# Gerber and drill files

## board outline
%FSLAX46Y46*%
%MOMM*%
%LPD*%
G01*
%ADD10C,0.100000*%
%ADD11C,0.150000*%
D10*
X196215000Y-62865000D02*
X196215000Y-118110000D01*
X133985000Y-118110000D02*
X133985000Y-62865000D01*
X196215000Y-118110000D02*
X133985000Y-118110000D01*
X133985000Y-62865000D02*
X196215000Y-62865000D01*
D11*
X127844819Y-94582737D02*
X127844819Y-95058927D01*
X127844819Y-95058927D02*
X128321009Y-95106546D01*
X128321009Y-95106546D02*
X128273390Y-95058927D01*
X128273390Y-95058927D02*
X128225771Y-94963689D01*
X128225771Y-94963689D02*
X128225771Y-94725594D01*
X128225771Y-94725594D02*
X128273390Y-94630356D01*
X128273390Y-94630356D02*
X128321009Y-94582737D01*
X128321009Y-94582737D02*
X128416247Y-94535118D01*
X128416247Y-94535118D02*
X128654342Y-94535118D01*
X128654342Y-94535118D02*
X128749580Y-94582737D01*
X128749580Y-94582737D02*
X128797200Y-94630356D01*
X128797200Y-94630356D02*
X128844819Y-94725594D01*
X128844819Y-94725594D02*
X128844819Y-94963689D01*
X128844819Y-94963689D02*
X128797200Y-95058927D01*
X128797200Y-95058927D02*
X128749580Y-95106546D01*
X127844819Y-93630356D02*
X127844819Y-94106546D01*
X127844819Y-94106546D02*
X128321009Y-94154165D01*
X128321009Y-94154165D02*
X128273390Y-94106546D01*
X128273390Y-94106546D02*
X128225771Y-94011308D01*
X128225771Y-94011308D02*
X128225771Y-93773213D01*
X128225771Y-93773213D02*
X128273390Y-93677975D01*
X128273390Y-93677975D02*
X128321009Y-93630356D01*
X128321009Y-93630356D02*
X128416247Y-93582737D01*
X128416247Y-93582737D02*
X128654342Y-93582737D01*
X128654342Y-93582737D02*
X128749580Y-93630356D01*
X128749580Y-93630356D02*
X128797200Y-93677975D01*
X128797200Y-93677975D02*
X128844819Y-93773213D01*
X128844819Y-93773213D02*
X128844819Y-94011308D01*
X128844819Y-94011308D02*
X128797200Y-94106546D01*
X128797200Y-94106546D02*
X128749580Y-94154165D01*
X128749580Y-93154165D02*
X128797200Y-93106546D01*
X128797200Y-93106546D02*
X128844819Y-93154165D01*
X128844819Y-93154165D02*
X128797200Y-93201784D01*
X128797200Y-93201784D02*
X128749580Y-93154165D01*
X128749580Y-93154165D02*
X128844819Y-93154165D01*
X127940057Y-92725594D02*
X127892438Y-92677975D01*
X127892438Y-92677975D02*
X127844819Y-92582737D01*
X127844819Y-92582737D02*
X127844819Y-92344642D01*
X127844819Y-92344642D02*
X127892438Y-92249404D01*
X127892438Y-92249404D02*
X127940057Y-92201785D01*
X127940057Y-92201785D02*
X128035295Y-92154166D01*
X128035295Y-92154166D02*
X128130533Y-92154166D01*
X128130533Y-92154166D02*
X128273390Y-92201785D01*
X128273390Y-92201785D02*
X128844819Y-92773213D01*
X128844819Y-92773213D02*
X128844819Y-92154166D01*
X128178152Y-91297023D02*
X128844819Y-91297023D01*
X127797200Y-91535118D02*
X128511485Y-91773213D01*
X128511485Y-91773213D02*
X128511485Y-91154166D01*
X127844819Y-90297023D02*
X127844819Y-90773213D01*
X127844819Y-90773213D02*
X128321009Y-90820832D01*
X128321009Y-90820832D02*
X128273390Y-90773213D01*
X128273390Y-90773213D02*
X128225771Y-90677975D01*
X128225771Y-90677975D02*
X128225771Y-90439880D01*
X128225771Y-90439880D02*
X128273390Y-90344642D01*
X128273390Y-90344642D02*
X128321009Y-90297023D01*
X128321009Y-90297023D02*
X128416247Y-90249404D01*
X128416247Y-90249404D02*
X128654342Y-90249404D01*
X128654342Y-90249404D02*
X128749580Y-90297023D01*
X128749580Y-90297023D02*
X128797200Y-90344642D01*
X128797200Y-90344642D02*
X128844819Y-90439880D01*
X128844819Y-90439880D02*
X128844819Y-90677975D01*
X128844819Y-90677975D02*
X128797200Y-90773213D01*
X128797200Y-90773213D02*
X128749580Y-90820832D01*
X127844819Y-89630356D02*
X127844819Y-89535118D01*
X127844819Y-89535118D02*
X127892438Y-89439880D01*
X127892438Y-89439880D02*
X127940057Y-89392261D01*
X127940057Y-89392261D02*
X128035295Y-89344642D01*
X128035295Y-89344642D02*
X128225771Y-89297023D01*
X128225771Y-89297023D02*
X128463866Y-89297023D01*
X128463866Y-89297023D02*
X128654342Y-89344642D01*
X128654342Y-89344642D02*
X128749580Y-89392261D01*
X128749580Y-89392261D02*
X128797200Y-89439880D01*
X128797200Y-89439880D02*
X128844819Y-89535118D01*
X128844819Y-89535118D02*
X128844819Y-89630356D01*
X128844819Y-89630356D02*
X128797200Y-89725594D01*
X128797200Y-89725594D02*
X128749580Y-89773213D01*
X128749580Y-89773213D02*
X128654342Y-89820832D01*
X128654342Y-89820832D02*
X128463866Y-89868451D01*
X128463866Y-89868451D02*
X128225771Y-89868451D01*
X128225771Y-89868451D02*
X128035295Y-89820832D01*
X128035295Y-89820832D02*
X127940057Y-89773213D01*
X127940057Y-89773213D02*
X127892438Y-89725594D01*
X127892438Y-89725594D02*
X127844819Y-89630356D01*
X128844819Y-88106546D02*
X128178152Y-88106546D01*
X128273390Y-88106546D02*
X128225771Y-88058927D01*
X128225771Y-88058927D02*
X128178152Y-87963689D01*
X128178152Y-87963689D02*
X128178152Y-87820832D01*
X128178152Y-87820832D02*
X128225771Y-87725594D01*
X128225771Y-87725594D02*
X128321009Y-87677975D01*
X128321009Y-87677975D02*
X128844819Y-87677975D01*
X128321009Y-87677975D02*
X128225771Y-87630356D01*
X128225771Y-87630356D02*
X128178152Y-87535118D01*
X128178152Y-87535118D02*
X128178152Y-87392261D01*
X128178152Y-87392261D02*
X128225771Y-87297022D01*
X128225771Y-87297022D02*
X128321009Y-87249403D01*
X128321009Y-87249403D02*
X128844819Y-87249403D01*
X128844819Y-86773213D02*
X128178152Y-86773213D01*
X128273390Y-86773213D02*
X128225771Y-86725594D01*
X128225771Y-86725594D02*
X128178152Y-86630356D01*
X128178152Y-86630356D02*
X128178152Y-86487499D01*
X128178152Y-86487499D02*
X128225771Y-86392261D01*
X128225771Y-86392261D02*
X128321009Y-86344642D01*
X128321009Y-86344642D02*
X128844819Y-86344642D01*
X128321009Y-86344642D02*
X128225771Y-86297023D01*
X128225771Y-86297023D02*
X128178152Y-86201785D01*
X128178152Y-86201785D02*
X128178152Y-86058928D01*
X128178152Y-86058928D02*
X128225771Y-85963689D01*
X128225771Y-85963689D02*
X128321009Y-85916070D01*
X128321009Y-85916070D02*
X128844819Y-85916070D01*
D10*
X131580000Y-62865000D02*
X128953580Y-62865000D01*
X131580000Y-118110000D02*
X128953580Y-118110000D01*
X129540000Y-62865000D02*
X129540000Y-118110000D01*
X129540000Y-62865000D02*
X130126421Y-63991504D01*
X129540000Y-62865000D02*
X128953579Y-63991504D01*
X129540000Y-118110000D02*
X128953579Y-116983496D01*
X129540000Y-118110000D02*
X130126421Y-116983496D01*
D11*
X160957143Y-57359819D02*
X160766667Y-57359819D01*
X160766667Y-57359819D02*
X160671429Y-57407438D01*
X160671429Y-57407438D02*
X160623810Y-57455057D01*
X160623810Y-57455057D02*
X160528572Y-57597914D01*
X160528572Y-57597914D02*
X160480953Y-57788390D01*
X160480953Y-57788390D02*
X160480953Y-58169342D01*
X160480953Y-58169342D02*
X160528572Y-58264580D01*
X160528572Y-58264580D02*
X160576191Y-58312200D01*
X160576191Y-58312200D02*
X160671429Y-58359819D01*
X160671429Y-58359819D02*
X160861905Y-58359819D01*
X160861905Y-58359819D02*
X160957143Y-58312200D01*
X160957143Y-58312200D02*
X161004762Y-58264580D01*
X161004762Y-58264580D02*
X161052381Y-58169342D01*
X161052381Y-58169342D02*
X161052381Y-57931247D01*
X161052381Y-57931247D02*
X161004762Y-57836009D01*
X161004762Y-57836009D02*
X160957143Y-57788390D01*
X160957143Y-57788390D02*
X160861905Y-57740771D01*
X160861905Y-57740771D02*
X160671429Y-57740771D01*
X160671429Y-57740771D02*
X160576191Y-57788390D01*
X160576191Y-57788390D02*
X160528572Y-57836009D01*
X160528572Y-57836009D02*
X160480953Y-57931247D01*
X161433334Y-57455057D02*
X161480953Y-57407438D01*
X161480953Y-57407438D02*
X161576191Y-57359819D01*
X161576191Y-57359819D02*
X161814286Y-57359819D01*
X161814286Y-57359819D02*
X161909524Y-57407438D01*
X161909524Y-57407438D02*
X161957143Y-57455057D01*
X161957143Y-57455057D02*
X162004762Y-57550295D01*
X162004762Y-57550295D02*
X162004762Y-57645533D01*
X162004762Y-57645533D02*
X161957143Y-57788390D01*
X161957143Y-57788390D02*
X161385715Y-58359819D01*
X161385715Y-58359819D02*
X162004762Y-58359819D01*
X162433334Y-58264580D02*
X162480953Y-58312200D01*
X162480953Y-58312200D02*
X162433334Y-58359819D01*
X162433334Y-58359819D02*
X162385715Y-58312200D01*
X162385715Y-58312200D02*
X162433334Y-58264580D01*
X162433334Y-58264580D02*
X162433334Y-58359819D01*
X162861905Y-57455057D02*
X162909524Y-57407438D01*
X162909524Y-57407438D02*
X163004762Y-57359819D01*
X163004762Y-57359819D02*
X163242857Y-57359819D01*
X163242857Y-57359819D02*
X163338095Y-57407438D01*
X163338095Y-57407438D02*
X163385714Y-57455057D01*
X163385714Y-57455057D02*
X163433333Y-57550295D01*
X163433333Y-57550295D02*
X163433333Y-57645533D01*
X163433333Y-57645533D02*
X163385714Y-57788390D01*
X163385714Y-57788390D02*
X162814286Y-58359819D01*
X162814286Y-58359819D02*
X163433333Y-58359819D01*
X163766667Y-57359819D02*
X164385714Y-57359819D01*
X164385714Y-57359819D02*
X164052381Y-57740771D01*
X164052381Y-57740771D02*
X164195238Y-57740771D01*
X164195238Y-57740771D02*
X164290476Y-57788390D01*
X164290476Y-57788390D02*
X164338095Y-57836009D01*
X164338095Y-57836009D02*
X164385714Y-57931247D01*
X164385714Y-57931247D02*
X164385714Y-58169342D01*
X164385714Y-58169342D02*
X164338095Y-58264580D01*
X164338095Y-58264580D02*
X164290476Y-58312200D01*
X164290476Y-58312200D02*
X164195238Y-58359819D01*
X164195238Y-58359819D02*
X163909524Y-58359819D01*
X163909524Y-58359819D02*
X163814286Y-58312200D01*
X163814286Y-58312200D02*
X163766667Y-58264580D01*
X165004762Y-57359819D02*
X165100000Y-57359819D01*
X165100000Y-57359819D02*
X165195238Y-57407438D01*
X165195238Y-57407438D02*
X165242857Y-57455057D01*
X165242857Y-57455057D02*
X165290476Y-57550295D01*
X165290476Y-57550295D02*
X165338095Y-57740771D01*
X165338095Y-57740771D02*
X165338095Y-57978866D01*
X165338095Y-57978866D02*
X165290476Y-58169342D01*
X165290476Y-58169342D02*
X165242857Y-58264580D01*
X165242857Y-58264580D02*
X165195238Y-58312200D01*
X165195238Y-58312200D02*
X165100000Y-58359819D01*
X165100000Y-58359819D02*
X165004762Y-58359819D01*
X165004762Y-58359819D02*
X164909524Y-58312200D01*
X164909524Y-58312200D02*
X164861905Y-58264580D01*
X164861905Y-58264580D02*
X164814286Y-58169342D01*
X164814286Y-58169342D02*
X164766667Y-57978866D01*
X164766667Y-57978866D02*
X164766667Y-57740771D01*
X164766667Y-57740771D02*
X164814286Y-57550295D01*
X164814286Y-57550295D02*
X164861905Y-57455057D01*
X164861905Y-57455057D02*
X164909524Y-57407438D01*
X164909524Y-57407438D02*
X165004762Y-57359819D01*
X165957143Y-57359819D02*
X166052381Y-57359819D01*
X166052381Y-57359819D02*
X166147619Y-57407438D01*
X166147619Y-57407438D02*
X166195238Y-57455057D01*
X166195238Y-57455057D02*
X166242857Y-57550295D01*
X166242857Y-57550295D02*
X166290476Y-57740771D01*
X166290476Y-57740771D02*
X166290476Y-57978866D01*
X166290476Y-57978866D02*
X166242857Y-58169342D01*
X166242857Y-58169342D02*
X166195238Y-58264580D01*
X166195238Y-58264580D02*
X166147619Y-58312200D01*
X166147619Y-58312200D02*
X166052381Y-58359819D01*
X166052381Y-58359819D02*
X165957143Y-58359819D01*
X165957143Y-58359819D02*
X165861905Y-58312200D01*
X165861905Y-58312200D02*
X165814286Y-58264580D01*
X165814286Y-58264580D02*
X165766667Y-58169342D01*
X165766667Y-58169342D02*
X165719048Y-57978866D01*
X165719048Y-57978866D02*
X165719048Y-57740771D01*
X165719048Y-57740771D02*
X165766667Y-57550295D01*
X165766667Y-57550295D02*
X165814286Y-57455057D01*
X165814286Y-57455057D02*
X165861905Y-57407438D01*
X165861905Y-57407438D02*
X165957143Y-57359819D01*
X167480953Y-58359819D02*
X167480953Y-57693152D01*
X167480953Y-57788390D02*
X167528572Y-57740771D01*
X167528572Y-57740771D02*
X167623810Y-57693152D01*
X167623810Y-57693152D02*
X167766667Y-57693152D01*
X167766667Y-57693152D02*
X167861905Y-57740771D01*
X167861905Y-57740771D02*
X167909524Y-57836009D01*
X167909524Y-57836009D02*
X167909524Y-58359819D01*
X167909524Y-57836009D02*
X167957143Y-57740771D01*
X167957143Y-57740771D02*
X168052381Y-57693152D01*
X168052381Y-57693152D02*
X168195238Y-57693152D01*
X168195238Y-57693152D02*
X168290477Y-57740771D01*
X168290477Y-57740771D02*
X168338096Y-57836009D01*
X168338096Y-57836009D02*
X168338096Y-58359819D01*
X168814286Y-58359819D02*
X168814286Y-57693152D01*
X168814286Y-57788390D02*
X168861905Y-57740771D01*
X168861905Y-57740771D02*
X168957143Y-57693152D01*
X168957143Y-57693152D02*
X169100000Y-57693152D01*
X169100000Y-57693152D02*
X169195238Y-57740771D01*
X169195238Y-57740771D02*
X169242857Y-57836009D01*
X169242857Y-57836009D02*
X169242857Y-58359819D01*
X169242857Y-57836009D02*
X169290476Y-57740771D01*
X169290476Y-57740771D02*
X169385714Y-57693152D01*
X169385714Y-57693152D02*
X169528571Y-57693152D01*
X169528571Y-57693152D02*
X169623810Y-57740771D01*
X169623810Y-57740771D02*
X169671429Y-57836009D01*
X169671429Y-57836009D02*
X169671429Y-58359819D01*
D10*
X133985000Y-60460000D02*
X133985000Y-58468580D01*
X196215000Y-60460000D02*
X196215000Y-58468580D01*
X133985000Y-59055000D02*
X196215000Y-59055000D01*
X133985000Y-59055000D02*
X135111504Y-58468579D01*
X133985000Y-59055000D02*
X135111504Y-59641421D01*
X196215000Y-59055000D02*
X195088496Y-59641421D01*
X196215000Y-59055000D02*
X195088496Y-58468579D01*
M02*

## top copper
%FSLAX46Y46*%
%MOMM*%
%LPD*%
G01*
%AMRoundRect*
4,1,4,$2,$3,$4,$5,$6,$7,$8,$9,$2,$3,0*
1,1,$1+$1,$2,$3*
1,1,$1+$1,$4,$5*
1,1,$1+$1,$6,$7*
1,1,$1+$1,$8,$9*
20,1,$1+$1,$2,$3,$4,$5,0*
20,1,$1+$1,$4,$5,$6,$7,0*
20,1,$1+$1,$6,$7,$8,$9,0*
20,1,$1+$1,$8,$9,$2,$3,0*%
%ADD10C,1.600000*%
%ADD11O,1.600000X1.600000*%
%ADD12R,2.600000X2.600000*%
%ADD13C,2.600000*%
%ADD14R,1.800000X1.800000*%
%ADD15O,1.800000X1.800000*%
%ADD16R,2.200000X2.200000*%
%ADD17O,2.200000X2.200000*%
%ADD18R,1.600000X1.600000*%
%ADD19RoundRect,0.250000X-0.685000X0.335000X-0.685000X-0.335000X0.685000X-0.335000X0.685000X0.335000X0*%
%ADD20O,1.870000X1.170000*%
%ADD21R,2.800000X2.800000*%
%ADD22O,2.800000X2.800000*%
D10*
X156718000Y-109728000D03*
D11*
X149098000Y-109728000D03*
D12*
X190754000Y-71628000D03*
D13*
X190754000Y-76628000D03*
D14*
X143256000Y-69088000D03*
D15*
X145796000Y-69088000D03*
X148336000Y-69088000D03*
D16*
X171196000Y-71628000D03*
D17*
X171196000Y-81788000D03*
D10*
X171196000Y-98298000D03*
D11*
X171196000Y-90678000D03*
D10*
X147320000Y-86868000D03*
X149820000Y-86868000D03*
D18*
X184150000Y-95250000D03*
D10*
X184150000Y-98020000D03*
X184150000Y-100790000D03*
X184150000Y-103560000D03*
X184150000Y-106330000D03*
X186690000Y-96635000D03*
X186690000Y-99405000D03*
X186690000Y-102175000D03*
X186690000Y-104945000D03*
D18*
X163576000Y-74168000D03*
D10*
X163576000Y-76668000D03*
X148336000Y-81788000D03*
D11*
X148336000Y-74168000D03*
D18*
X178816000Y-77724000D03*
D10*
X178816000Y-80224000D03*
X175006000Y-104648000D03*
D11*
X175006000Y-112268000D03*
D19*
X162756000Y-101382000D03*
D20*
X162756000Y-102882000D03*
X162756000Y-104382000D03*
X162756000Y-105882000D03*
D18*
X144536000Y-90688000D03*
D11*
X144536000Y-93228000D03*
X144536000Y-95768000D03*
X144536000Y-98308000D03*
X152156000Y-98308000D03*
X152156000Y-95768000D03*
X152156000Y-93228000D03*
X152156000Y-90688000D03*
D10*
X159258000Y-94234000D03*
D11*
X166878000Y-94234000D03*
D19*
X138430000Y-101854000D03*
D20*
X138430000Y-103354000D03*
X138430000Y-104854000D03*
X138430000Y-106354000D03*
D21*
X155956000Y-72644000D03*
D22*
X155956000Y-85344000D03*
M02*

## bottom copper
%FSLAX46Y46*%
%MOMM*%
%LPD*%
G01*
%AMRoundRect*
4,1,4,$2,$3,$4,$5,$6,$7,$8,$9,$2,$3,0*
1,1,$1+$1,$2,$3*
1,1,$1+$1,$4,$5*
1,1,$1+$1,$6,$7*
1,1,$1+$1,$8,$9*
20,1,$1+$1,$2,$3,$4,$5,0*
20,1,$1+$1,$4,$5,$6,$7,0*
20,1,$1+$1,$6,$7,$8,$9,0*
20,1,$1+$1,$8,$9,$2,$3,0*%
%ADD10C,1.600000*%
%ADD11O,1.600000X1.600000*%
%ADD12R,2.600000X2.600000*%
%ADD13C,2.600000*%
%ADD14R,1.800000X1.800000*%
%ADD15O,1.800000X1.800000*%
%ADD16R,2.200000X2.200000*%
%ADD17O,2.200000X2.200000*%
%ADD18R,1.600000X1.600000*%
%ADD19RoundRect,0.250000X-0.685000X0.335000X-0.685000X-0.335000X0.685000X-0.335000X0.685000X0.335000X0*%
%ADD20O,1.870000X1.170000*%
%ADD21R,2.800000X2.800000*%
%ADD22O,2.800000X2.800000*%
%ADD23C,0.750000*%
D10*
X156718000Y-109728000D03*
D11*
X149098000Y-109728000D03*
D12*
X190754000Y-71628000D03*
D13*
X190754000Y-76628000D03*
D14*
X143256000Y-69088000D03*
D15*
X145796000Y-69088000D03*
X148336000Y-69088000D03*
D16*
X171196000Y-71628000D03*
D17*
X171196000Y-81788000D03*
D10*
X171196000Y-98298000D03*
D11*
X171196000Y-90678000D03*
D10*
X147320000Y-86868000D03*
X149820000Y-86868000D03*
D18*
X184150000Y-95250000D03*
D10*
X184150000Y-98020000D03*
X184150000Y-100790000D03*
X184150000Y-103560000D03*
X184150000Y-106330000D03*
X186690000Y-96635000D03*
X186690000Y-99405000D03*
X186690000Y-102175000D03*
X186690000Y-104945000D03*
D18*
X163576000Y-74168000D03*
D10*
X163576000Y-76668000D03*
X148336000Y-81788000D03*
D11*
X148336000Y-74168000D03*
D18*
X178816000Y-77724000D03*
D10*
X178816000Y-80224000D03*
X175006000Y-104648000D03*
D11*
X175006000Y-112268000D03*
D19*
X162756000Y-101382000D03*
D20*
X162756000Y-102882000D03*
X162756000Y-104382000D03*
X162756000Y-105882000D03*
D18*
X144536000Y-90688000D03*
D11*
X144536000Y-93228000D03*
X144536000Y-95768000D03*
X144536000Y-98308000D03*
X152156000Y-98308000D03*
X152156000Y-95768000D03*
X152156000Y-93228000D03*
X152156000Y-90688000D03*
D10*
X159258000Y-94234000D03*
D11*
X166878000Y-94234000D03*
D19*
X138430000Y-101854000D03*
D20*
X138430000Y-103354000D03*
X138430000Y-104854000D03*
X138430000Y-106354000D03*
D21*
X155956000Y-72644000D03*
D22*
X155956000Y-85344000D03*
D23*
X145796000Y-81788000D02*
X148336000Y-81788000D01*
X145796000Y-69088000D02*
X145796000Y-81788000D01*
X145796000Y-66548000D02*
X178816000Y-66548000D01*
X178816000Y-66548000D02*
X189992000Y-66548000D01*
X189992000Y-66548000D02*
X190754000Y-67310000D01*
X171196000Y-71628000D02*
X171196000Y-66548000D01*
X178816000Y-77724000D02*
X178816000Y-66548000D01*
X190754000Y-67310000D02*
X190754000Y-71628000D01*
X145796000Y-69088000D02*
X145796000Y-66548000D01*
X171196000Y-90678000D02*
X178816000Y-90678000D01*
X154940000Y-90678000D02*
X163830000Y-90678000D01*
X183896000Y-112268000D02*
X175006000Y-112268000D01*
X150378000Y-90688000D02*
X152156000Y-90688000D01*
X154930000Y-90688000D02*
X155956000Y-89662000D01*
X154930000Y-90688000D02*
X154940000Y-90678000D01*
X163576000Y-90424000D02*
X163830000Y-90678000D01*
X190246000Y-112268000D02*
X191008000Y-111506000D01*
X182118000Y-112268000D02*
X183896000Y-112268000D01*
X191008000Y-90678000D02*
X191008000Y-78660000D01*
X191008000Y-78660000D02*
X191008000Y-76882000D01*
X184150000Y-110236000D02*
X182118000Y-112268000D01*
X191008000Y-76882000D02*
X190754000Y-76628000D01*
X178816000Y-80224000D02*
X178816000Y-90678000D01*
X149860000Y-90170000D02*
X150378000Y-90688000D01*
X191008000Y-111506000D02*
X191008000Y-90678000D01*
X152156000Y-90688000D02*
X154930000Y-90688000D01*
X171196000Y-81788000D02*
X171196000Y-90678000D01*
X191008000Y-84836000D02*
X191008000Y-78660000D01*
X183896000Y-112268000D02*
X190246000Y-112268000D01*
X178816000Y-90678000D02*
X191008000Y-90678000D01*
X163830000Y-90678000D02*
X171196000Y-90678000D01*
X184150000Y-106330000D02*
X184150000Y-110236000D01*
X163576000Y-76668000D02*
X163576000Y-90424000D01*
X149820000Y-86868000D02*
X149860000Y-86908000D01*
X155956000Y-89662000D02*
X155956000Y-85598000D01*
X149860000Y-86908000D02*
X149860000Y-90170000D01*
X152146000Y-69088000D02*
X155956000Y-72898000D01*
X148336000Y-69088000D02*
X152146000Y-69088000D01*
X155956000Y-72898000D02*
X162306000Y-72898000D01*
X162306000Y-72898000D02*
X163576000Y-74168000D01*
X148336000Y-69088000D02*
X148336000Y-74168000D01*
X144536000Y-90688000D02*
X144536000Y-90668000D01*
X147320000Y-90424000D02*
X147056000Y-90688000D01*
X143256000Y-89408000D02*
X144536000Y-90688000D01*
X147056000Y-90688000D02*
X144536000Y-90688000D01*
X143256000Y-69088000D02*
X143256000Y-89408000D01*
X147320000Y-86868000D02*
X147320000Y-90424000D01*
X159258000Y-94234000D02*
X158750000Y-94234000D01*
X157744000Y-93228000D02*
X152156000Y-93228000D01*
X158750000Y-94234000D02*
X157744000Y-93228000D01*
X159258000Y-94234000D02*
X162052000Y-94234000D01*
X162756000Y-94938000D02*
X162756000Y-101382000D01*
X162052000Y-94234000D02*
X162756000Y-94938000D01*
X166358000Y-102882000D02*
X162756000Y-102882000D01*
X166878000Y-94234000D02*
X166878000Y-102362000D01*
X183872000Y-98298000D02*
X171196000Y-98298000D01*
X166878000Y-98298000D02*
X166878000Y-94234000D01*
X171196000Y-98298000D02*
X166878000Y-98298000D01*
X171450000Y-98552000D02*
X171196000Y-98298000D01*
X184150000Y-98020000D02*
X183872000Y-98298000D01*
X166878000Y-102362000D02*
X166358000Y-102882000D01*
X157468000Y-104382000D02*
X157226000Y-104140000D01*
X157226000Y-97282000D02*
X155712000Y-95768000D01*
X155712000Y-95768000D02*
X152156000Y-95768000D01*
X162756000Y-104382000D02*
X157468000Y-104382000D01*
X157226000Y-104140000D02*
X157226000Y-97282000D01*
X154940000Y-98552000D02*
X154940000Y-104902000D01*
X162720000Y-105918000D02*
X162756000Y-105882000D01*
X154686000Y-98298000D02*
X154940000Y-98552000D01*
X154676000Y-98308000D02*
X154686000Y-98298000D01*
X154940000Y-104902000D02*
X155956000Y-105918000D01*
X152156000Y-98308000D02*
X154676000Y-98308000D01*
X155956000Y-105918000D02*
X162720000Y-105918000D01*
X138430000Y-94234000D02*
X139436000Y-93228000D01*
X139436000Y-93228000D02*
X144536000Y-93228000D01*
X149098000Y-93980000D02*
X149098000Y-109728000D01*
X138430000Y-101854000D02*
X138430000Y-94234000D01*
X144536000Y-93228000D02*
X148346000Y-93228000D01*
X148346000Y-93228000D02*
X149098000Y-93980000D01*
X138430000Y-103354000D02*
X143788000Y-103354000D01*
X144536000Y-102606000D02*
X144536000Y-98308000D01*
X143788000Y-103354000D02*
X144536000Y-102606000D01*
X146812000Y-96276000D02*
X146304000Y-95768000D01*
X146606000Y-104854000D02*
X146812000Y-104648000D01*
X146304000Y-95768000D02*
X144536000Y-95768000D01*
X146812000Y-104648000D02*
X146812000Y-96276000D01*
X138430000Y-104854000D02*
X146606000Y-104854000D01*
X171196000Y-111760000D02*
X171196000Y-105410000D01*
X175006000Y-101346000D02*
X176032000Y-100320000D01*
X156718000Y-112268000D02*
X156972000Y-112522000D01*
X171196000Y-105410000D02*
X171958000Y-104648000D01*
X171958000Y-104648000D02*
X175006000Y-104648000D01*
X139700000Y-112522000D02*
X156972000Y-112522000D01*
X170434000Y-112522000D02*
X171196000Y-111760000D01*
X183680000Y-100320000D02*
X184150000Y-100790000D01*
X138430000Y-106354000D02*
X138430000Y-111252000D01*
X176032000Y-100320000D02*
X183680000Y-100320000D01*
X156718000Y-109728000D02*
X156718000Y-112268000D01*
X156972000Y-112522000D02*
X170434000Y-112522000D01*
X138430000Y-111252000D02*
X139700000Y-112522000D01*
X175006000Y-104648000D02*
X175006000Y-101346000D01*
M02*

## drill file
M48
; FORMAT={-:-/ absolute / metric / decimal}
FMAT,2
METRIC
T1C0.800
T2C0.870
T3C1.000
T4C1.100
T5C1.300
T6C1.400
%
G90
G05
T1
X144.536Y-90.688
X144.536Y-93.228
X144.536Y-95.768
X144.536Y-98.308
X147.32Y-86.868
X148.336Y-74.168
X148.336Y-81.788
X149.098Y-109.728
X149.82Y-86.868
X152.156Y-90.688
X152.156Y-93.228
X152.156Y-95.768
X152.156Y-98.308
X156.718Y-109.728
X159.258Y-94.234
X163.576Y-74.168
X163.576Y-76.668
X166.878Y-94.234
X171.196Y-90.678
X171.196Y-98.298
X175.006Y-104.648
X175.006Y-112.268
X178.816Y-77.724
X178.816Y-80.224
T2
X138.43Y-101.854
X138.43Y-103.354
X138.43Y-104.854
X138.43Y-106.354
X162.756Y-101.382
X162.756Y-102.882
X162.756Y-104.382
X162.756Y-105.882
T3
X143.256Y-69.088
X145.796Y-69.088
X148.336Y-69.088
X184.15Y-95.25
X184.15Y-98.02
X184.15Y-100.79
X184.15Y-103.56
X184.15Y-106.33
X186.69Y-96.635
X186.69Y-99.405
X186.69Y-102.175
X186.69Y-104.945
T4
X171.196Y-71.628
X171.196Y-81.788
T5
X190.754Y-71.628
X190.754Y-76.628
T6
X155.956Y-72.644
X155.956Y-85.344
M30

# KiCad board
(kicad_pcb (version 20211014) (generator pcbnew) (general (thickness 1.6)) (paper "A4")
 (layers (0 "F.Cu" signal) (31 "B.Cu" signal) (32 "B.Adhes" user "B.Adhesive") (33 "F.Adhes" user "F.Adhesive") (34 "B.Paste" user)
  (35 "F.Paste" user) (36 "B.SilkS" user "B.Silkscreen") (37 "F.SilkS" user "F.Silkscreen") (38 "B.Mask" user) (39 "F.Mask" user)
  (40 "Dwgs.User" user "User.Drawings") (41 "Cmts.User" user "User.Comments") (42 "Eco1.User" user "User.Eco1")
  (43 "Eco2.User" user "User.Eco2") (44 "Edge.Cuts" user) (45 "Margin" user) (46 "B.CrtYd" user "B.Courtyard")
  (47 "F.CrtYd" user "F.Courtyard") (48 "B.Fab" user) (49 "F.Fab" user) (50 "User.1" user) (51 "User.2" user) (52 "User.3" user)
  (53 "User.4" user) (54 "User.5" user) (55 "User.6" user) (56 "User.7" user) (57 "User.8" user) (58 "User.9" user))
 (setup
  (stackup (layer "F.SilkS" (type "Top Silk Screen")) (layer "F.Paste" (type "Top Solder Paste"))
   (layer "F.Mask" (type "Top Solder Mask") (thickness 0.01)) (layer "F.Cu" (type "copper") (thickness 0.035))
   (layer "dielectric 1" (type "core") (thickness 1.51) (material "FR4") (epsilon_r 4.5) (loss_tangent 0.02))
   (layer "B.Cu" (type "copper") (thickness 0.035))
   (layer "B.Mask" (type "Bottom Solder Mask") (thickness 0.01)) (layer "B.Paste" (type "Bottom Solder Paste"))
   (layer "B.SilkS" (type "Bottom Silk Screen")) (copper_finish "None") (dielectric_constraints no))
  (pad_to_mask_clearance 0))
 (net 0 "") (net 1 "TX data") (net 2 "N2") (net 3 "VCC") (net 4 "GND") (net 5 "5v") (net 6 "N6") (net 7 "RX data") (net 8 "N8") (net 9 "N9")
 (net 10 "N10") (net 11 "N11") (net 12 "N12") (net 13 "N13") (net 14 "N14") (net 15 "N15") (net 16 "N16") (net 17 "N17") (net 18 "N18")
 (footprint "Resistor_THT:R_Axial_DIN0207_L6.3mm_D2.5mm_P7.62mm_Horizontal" (layer "F.Cu") (at 156.718 109.728 180)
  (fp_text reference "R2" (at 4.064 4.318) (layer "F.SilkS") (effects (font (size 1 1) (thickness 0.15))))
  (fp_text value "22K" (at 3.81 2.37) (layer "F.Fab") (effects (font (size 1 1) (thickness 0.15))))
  (pad "1" thru_hole circle (at 0 0 180) (size 1.6 1.6) (drill 0.8) (layers *.Cu *.Mask) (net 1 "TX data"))
  (pad "2" thru_hole oval (at 7.62 0 180) (size 1.6 1.6) (drill 0.8) (layers *.Cu *.Mask) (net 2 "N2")))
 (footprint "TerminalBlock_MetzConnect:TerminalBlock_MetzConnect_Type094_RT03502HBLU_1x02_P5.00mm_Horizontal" (layer "F.Cu")
  (at 190.754 71.628 -90)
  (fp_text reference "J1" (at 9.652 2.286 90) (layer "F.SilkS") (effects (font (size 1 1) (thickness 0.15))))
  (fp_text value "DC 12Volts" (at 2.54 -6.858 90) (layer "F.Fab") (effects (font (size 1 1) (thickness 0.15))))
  (pad "1" thru_hole rect (at 0 0 270) (size 2.6 2.6) (drill 1.3) (layers *.Cu *.Mask) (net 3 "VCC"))
  (pad "2" thru_hole circle (at 5 0 270) (size 2.6 2.6) (drill 1.3) (layers *.Cu *.Mask) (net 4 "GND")))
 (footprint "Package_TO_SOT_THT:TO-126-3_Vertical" (layer "F.Cu") (at 143.256 69.088)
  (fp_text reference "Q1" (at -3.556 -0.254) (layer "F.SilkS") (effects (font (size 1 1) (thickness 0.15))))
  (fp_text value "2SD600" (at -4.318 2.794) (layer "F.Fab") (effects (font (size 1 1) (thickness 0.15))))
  (pad "1" thru_hole rect (at 0 0) (size 1.8 1.8) (drill 1) (layers *.Cu *.Mask) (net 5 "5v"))
  (pad "2" thru_hole oval (at 2.54 0) (size 1.8 1.8) (drill 1) (layers *.Cu *.Mask) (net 3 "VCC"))
  (pad "3" thru_hole oval (at 5.08 0) (size 1.8 1.8) (drill 1) (layers *.Cu *.Mask) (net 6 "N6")))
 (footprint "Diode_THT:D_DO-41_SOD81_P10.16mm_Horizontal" (layer "F.Cu") (at 171.196 71.628 -90)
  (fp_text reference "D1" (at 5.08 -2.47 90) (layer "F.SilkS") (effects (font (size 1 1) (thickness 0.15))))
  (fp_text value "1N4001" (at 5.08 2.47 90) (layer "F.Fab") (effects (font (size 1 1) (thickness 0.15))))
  (pad "1" thru_hole rect (at 0 0 270) (size 2.2 2.2) (drill 1.1) (layers *.Cu *.Mask) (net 3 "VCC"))
  (pad "2" thru_hole oval (at 10.16 0 270) (size 2.2 2.2) (drill 1.1) (layers *.Cu *.Mask) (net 4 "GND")))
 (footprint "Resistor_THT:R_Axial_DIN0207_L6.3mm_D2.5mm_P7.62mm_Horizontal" (layer "F.Cu") (at 171.196 98.298 90)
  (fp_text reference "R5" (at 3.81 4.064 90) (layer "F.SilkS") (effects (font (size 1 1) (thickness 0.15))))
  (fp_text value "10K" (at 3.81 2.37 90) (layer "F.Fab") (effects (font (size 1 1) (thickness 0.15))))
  (pad "1" thru_hole circle (at 0 0 90) (size 1.6 1.6) (drill 0.8) (layers *.Cu *.Mask) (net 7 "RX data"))
  (pad "2" thru_hole oval (at 7.62 0 90) (size 1.6 1.6) (drill 0.8) (layers *.Cu *.Mask) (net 4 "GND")))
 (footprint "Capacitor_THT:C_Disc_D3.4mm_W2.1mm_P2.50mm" (layer "F.Cu") (at 147.32 86.868)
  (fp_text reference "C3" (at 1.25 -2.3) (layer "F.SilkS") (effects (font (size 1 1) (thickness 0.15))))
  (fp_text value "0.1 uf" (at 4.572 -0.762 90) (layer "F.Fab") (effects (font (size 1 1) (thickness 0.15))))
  (pad "1" thru_hole circle (at 0 0) (size 1.6 1.6) (drill 0.8) (layers *.Cu *.Mask) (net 5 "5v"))
  (pad "2" thru_hole circle (at 2.5 0) (size 1.6 1.6) (drill 0.8) (layers *.Cu *.Mask) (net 4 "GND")))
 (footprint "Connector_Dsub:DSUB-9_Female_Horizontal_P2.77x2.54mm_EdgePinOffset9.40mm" (layer "F.Cu") (at 184.15 95.25 90)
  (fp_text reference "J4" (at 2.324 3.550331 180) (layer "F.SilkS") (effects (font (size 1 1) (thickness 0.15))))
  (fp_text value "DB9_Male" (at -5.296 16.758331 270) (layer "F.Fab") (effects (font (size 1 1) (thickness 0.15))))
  (pad "1" thru_hole rect (at 0 0 90) (size 1.6 1.6) (drill 1) (layers *.Cu *.Mask) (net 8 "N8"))
  (pad "2" thru_hole circle (at -2.77 0 90) (size 1.6 1.6) (drill 1) (layers *.Cu *.Mask) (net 7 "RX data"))
  (pad "3" thru_hole circle (at -5.54 0 90) (size 1.6 1.6) (drill 1) (layers *.Cu *.Mask) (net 1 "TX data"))
  (pad "4" thru_hole circle (at -8.31 0 90) (size 1.6 1.6) (drill 1) (layers *.Cu *.Mask) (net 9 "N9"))
  (pad "5" thru_hole circle (at -11.08 0 90) (size 1.6 1.6) (drill 1) (layers *.Cu *.Mask) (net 4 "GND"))
  (pad "6" thru_hole circle (at -1.385 2.54 90) (size 1.6 1.6) (drill 1) (layers *.Cu *.Mask) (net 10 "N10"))
  (pad "7" thru_hole circle (at -4.155 2.54 90) (size 1.6 1.6) (drill 1) (layers *.Cu *.Mask) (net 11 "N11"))
  (pad "8" thru_hole circle (at -6.925 2.54 90) (size 1.6 1.6) (drill 1) (layers *.Cu *.Mask) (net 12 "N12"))
  (pad "9" thru_hole circle (at -9.695 2.54 90) (size 1.6 1.6) (drill 1) (layers *.Cu *.Mask) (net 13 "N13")))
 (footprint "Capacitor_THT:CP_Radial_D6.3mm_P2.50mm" (layer "F.Cu") (at 163.576 74.168 -90)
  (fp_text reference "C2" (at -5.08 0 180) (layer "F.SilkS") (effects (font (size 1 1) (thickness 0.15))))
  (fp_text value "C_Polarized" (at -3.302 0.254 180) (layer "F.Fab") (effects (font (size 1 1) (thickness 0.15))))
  (pad "1" thru_hole rect (at 0 0 270) (size 1.6 1.6) (drill 0.8) (layers *.Cu *.Mask) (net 6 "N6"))
  (pad "2" thru_hole circle (at 2.5 0 270) (size 1.6 1.6) (drill 0.8) (layers *.Cu *.Mask) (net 4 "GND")))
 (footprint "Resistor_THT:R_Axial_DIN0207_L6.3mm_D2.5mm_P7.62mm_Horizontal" (layer "F.Cu") (at 148.336 81.788 90)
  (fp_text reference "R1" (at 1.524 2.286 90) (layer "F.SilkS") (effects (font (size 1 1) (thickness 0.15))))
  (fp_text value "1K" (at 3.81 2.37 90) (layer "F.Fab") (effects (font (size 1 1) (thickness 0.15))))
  (pad "1" thru_hole circle (at 0 0 90) (size 1.6 1.6) (drill 0.8) (layers *.Cu *.Mask) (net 3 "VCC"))
  (pad "2" thru_hole oval (at 7.62 0 90) (size 1.6 1.6) (drill 0.8) (layers *.Cu *.Mask) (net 6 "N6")))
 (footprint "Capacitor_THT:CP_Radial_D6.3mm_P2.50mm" (layer "F.Cu") (at 178.816 77.724 -90)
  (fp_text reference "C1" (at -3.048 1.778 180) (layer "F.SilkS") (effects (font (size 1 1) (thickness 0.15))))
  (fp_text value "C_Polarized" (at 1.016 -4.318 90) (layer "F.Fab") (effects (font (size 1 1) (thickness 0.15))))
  (pad "1" thru_hole rect (at 0 0 270) (size 1.6 1.6) (drill 0.8) (layers *.Cu *.Mask) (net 3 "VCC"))
  (pad "2" thru_hole circle (at 2.5 0 270) (size 1.6 1.6) (drill 0.8) (layers *.Cu *.Mask) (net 4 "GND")))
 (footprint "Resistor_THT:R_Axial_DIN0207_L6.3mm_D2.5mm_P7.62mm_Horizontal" (layer "F.Cu") (at 175.006 104.648 -90)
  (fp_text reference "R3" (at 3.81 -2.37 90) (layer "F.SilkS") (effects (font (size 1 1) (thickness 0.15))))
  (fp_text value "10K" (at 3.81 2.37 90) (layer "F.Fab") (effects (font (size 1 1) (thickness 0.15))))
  (pad "1" thru_hole circle (at 0 0 270) (size 1.6 1.6) (drill 0.8) (layers *.Cu *.Mask) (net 1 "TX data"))
  (pad "2" thru_hole oval (at 7.62 0 270) (size 1.6 1.6) (drill 0.8) (layers *.Cu *.Mask) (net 4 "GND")))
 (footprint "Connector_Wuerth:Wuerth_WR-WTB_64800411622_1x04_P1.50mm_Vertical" (layer "F.Cu") (at 162.756 101.382 -90)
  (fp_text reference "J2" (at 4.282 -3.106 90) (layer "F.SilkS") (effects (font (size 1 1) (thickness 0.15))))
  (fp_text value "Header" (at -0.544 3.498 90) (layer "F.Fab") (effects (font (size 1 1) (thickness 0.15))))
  (pad "1" thru_hole roundrect (at 0 0 270) (size 1.17 1.87) (drill 0.87) (layers *.Cu *.Mask) (roundrect_rratio 0.213675) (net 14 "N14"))
  (pad "2" thru_hole oval (at 1.5 0 270) (size 1.17 1.87) (drill 0.87) (layers *.Cu *.Mask) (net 7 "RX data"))
  (pad "3" thru_hole oval (at 3 0 270) (size 1.17 1.87) (drill 0.87) (layers *.Cu *.Mask) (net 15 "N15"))
  (pad "4" thru_hole oval (at 4.5 0 270) (size 1.17 1.87) (drill 0.87) (layers *.Cu *.Mask) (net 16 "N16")))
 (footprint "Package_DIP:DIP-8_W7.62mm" (layer "F.Cu") (at 144.536 90.688)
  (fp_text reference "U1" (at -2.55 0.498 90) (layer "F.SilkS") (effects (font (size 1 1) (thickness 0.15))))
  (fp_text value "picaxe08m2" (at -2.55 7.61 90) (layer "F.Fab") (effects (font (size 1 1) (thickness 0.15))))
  (pad "1" thru_hole rect (at 0 0) (size 1.6 1.6) (drill 0.8) (layers *.Cu *.Mask) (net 5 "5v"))
  (pad "2" thru_hole oval (at 0 2.54) (size 1.6 1.6) (drill 0.8) (layers *.Cu *.Mask) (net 2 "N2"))
  (pad "3" thru_hole oval (at 0 5.08) (size 1.6 1.6) (drill 0.8) (layers *.Cu *.Mask) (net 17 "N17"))
  (pad "4" thru_hole oval (at 0 7.62) (size 1.6 1.6) (drill 0.8) (layers *.Cu *.Mask) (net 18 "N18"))
  (pad "5" thru_hole oval (at 7.62 7.62) (size 1.6 1.6) (drill 0.8) (layers *.Cu *.Mask) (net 16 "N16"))
  (pad "6" thru_hole oval (at 7.62 5.08) (size 1.6 1.6) (drill 0.8) (layers *.Cu *.Mask) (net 15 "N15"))
  (pad "7" thru_hole oval (at 7.62 2.54) (size 1.6 1.6) (drill 0.8) (layers *.Cu *.Mask) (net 14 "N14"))
  (pad "8" thru_hole oval (at 7.62 0) (size 1.6 1.6) (drill 0.8) (layers *.Cu *.Mask) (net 4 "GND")))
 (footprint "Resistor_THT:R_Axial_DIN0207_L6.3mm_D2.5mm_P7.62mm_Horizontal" (layer "F.Cu") (at 159.258 94.234)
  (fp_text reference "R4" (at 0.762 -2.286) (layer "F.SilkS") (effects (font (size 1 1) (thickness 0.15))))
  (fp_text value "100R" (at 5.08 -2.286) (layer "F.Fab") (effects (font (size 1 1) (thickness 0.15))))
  (pad "1" thru_hole circle (at 0 0) (size 1.6 1.6) (drill 0.8) (layers *.Cu *.Mask) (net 14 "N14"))
  (pad "2" thru_hole oval (at 7.62 0) (size 1.6 1.6) (drill 0.8) (layers *.Cu *.Mask) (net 7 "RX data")))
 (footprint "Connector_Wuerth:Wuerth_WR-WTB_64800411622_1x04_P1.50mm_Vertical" (layer "F.Cu") (at 138.43 101.854 -90)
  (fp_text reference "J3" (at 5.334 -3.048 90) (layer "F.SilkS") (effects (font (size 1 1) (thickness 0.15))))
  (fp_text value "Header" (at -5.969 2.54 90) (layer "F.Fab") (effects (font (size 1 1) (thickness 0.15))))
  (pad "1" thru_hole roundrect (at 0 0 270) (size 1.17 1.87) (drill 0.87) (layers *.Cu *.Mask) (roundrect_rratio 0.213675) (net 2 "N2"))
  (pad "2" thru_hole oval (at 1.5 0 270) (size 1.17 1.87) (drill 0.87) (layers *.Cu *.Mask) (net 18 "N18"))
  (pad "3" thru_hole oval (at 3 0 270) (size 1.17 1.87) (drill 0.87) (layers *.Cu *.Mask) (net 17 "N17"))
  (pad "4" thru_hole oval (at 4.5 0 270) (size 1.17 1.87) (drill 0.87) (layers *.Cu *.Mask) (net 1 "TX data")))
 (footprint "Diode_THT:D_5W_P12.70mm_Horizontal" (layer "F.Cu") (at 155.956 72.644 -90)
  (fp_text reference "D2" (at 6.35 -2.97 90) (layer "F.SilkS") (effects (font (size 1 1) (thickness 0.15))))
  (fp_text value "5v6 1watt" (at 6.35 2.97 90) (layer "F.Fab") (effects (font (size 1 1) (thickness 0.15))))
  (pad "1" thru_hole rect (at 0 0 270) (size 2.8 2.8) (drill 1.4) (layers *.Cu *.Mask) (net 6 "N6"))
  (pad "2" thru_hole oval (at 12.7 0 270) (size 2.8 2.8) (drill 1.4) (layers *.Cu *.Mask) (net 4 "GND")))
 (gr_line (start 196.215 62.865) (end 196.215 118.11) (layer "Edge.Cuts") (width 0.1))
 (gr_line (start 133.985 118.11) (end 133.985 62.865) (layer "Edge.Cuts") (width 0.1))
 (gr_line (start 196.215 118.11) (end 133.985 118.11) (layer "Edge.Cuts") (width 0.1))
 (gr_line (start 133.985 62.865) (end 196.215 62.865) (layer "Edge.Cuts") (width 0.1))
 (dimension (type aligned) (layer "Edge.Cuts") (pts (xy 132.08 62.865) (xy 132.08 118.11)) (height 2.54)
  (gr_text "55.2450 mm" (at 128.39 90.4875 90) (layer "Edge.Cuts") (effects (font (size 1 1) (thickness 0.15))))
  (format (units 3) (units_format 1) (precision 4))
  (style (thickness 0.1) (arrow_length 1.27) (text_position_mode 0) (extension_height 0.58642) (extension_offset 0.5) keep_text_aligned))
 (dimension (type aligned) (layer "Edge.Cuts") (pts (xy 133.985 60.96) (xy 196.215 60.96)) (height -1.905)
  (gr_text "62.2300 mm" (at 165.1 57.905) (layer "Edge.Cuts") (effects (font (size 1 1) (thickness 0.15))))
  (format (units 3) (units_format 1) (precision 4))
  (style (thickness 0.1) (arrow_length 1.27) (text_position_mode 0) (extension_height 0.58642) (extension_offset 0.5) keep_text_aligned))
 (segment (start 145.796 81.788) (end 148.336 81.788) (width 0.75) (layer "B.Cu") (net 3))
 (segment (start 145.796 69.088) (end 145.796 81.788) (width 0.75) (layer "B.Cu") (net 3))
 (segment (start 145.796 66.548) (end 178.816 66.548) (width 0.75) (layer "B.Cu") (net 3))
 (segment (start 178.816 66.548) (end 189.992 66.548) (width 0.75) (layer "B.Cu") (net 3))
 (segment (start 189.992 66.548) (end 190.754 67.31) (width 0.75) (layer "B.Cu") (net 3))
 (segment (start 171.196 71.628) (end 171.196 66.548) (width 0.75) (layer "B.Cu") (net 3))
 (segment (start 178.816 77.724) (end 178.816 66.548) (width 0.75) (layer "B.Cu") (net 3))
 (segment (start 190.754 67.31) (end 190.754 71.628) (width 0.75) (layer "B.Cu") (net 3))
 (segment (start 145.796 69.088) (end 145.796 66.548) (width 0.75) (layer "B.Cu") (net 3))
 (segment (start 171.196 90.678) (end 178.816 90.678) (width 0.75) (layer "B.Cu") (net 4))
 (segment (start 154.94 90.678) (end 163.83 90.678) (width 0.75) (layer "B.Cu") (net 4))
 (segment (start 183.896 112.268) (end 175.006 112.268) (width 0.75) (layer "B.Cu") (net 4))
 (segment (start 150.378 90.688) (end 152.156 90.688) (width 0.75) (layer "B.Cu") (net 4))
 (segment (start 154.93 90.688) (end 155.956 89.662) (width 0.75) (layer "B.Cu") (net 4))
 (segment (start 154.93 90.688) (end 154.94 90.678) (width 0.75) (layer "B.Cu") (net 4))
 (segment (start 163.576 90.424) (end 163.83 90.678) (width 0.75) (layer "B.Cu") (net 4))
 (segment (start 190.246 112.268) (end 191.008 111.506) (width 0.75) (layer "B.Cu") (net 4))
 (segment (start 182.118 112.268) (end 183.896 112.268) (width 0.75) (layer "B.Cu") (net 4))
 (segment (start 191.008 90.678) (end 191.008 78.66) (width 0.75) (layer "B.Cu") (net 4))
 (segment (start 191.008 78.66) (end 191.008 76.882) (width 0.75) (layer "B.Cu") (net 4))
 (segment (start 184.15 110.236) (end 182.118 112.268) (width 0.75) (layer "B.Cu") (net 4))
 (segment (start 191.008 76.882) (end 190.754 76.628) (width 0.75) (layer "B.Cu") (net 4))
 (segment (start 178.816 80.224) (end 178.816 90.678) (width 0.75) (layer "B.Cu") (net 4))
 (segment (start 149.86 90.17) (end 150.378 90.688) (width 0.75) (layer "B.Cu") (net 4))
 (segment (start 191.008 111.506) (end 191.008 90.678) (width 0.75) (layer "B.Cu") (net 4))
 (segment (start 152.156 90.688) (end 154.93 90.688) (width 0.75) (layer "B.Cu") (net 4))
 (segment (start 171.196 81.788) (end 171.196 90.678) (width 0.75) (layer "B.Cu") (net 4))
 (segment (start 191.008 84.836) (end 191.008 78.66) (width 0.75) (layer "B.Cu") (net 4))
 (segment (start 183.896 112.268) (end 190.246 112.268) (width 0.75) (layer "B.Cu") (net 4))
 (segment (start 178.816 90.678) (end 191.008 90.678) (width 0.75) (layer "B.Cu") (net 4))
 (segment (start 163.83 90.678) (end 171.196 90.678) (width 0.75) (layer "B.Cu") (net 4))
 (segment (start 184.15 106.33) (end 184.15 110.236) (width 0.75) (layer "B.Cu") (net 4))
 (segment (start 163.576 76.668) (end 163.576 90.424) (width 0.75) (layer "B.Cu") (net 4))
 (segment (start 149.82 86.868) (end 149.86 86.908) (width 0.75) (layer "B.Cu") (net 4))
 (segment (start 155.956 89.662) (end 155.956 85.598) (width 0.75) (layer "B.Cu") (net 4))
 (segment (start 149.86 86.908) (end 149.86 90.17) (width 0.75) (layer "B.Cu") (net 4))
 (segment (start 152.146 69.088) (end 155.956 72.898) (width 0.75) (layer "B.Cu") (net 6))
 (segment (start 148.336 69.088) (end 152.146 69.088) (width 0.75) (layer "B.Cu") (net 6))
 (segment (start 155.956 72.898) (end 162.306 72.898) (width 0.75) (layer "B.Cu") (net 6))
 (segment (start 162.306 72.898) (end 163.576 74.168) (width 0.75) (layer "B.Cu") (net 6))
 (segment (start 148.336 69.088) (end 148.336 74.168) (width 0.75) (layer "B.Cu") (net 6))
 (segment (start 144.536 90.688) (end 144.536 90.668) (width 0.75) (layer "B.Cu") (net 5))
 (segment (start 147.32 90.424) (end 147.056 90.688) (width 0.75) (layer "B.Cu") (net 5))
 (segment (start 143.256 89.408) (end 144.536 90.688) (width 0.75) (layer "B.Cu") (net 5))
 (segment (start 147.056 90.688) (end 144.536 90.688) (width 0.75) (layer "B.Cu") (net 5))
 (segment (start 143.256 69.088) (end 143.256 89.408) (width 0.75) (layer "B.Cu") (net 5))
 (segment (start 147.32 86.868) (end 147.32 90.424) (width 0.75) (layer "B.Cu") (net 5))
 (segment (start 159.258 94.234) (end 158.75 94.234) (width 0.75) (layer "B.Cu") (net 14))
 (segment (start 157.744 93.228) (end 152.156 93.228) (width 0.75) (layer "B.Cu") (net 14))
 (segment (start 158.75 94.234) (end 157.744 93.228) (width 0.75) (layer "B.Cu") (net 14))
 (segment (start 159.258 94.234) (end 162.052 94.234) (width 0.75) (layer "B.Cu") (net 14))
 (segment (start 162.756 94.938) (end 162.756 101.382) (width 0.75) (layer "B.Cu") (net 14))
 (segment (start 162.052 94.234) (end 162.756 94.938) (width 0.75) (layer "B.Cu") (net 14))
 (segment (start 166.358 102.882) (end 162.756 102.882) (width 0.75) (layer "B.Cu") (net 7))
 (segment (start 166.878 94.234) (end 166.878 102.362) (width 0.75) (layer "B.Cu") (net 7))
 (segment (start 183.872 98.298) (end 171.196 98.298) (width 0.75) (layer "B.Cu") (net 7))
 (segment (start 166.878 98.298) (end 166.878 94.234) (width 0.75) (layer "B.Cu") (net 7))
 (segment (start 171.196 98.298) (end 166.878 98.298) (width 0.75) (layer "B.Cu") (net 7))
 (segment (start 171.45 98.552) (end 171.196 98.298) (width 0.75) (layer "B.Cu") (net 7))
 (segment (start 184.15 98.02) (end 183.872 98.298) (width 0.75) (layer "B.Cu") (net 7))
 (segment (start 166.878 102.362) (end 166.358 102.882) (width 0.75) (layer "B.Cu") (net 7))
 (segment (start 157.468 104.382) (end 157.226 104.14) (width 0.75) (layer "B.Cu") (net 15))
 (segment (start 157.226 97.282) (end 155.712 95.768) (width 0.75) (layer "B.Cu") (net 15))
 (segment (start 155.712 95.768) (end 152.156 95.768) (width 0.75) (layer "B.Cu") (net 15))
 (segment (start 162.756 104.382) (end 157.468 104.382) (width 0.75) (layer "B.Cu") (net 15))
 (segment (start 157.226 104.14) (end 157.226 97.282) (width 0.75) (layer "B.Cu") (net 15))
 (segment (start 154.94 98.552) (end 154.94 104.902) (width 0.75) (layer "B.Cu") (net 16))
 (segment (start 162.72 105.918) (end 162.756 105.882) (width 0.75) (layer "B.Cu") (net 16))
 (segment (start 154.686 98.298) (end 154.94 98.552) (width 0.75) (layer "B.Cu") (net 16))
 (segment (start 154.676 98.308) (end 154.686 98.298) (width 0.75) (layer "B.Cu") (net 16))
 (segment (start 154.94 104.902) (end 155.956 105.918) (width 0.75) (layer "B.Cu") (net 16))
 (segment (start 152.156 98.308) (end 154.676 98.308) (width 0.75) (layer "B.Cu") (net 16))
 (segment (start 155.956 105.918) (end 162.72 105.918) (width 0.75) (layer "B.Cu") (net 16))
 (segment (start 138.43 94.234) (end 139.436 93.228) (width 0.75) (layer "B.Cu") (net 2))
 (segment (start 139.436 93.228) (end 144.536 93.228) (width 0.75) (layer "B.Cu") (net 2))
 (segment (start 149.098 93.98) (end 149.098 109.728) (width 0.75) (layer "B.Cu") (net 2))
 (segment (start 138.43 101.854) (end 138.43 94.234) (width 0.75) (layer "B.Cu") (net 2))
 (segment (start 144.536 93.228) (end 148.346 93.228) (width 0.75) (layer "B.Cu") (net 2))
 (segment (start 148.346 93.228) (end 149.098 93.98) (width 0.75) (layer "B.Cu") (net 2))
 (segment (start 138.43 103.354) (end 143.788 103.354) (width 0.75) (layer "B.Cu") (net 18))
 (segment (start 144.536 102.606) (end 144.536 98.308) (width 0.75) (layer "B.Cu") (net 18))
 (segment (start 143.788 103.354) (end 144.536 102.606) (width 0.75) (layer "B.Cu") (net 18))
 (segment (start 146.812 96.276) (end 146.304 95.768) (width 0.75) (layer "B.Cu") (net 17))
 (segment (start 146.606 104.854) (end 146.812 104.648) (width 0.75) (layer "B.Cu") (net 17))
 (segment (start 146.304 95.768) (end 144.536 95.768) (width 0.75) (layer "B.Cu") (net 17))
 (segment (start 146.812 104.648) (end 146.812 96.276) (width 0.75) (layer "B.Cu") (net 17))
 (segment (start 138.43 104.854) (end 146.606 104.854) (width 0.75) (layer "B.Cu") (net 17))
 (segment (start 171.196 111.76) (end 171.196 105.41) (width 0.75) (layer "B.Cu") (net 1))
 (segment (start 175.006 101.346) (end 176.032 100.32) (width 0.75) (layer "B.Cu") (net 1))
 (segment (start 156.718 112.268) (end 156.972 112.522) (width 0.75) (layer "B.Cu") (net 1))
 (segment (start 171.196 105.41) (end 171.958 104.648) (width 0.75) (layer "B.Cu") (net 1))
 (segment (start 171.958 104.648) (end 175.006 104.648) (width 0.75) (layer "B.Cu") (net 1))
 (segment (start 139.7 112.522) (end 156.972 112.522) (width 0.75) (layer "B.Cu") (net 1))
 (segment (start 170.434 112.522) (end 171.196 111.76) (width 0.75) (layer "B.Cu") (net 1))
 (segment (start 183.68 100.32) (end 184.15 100.79) (width 0.75) (layer "B.Cu") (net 1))
 (segment (start 138.43 106.354) (end 138.43 111.252) (width 0.75) (layer "B.Cu") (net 1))
 (segment (start 176.032 100.32) (end 183.68 100.32) (width 0.75) (layer "B.Cu") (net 1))
 (segment (start 156.718 109.728) (end 156.718 112.268) (width 0.75) (layer "B.Cu") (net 1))
 (segment (start 156.972 112.522) (end 170.434 112.522) (width 0.75) (layer "B.Cu") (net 1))
 (segment (start 138.43 111.252) (end 139.7 112.522) (width 0.75) (layer "B.Cu") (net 1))
 (segment (start 175.006 104.648) (end 175.006 101.346) (width 0.75) (layer "B.Cu") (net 1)))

